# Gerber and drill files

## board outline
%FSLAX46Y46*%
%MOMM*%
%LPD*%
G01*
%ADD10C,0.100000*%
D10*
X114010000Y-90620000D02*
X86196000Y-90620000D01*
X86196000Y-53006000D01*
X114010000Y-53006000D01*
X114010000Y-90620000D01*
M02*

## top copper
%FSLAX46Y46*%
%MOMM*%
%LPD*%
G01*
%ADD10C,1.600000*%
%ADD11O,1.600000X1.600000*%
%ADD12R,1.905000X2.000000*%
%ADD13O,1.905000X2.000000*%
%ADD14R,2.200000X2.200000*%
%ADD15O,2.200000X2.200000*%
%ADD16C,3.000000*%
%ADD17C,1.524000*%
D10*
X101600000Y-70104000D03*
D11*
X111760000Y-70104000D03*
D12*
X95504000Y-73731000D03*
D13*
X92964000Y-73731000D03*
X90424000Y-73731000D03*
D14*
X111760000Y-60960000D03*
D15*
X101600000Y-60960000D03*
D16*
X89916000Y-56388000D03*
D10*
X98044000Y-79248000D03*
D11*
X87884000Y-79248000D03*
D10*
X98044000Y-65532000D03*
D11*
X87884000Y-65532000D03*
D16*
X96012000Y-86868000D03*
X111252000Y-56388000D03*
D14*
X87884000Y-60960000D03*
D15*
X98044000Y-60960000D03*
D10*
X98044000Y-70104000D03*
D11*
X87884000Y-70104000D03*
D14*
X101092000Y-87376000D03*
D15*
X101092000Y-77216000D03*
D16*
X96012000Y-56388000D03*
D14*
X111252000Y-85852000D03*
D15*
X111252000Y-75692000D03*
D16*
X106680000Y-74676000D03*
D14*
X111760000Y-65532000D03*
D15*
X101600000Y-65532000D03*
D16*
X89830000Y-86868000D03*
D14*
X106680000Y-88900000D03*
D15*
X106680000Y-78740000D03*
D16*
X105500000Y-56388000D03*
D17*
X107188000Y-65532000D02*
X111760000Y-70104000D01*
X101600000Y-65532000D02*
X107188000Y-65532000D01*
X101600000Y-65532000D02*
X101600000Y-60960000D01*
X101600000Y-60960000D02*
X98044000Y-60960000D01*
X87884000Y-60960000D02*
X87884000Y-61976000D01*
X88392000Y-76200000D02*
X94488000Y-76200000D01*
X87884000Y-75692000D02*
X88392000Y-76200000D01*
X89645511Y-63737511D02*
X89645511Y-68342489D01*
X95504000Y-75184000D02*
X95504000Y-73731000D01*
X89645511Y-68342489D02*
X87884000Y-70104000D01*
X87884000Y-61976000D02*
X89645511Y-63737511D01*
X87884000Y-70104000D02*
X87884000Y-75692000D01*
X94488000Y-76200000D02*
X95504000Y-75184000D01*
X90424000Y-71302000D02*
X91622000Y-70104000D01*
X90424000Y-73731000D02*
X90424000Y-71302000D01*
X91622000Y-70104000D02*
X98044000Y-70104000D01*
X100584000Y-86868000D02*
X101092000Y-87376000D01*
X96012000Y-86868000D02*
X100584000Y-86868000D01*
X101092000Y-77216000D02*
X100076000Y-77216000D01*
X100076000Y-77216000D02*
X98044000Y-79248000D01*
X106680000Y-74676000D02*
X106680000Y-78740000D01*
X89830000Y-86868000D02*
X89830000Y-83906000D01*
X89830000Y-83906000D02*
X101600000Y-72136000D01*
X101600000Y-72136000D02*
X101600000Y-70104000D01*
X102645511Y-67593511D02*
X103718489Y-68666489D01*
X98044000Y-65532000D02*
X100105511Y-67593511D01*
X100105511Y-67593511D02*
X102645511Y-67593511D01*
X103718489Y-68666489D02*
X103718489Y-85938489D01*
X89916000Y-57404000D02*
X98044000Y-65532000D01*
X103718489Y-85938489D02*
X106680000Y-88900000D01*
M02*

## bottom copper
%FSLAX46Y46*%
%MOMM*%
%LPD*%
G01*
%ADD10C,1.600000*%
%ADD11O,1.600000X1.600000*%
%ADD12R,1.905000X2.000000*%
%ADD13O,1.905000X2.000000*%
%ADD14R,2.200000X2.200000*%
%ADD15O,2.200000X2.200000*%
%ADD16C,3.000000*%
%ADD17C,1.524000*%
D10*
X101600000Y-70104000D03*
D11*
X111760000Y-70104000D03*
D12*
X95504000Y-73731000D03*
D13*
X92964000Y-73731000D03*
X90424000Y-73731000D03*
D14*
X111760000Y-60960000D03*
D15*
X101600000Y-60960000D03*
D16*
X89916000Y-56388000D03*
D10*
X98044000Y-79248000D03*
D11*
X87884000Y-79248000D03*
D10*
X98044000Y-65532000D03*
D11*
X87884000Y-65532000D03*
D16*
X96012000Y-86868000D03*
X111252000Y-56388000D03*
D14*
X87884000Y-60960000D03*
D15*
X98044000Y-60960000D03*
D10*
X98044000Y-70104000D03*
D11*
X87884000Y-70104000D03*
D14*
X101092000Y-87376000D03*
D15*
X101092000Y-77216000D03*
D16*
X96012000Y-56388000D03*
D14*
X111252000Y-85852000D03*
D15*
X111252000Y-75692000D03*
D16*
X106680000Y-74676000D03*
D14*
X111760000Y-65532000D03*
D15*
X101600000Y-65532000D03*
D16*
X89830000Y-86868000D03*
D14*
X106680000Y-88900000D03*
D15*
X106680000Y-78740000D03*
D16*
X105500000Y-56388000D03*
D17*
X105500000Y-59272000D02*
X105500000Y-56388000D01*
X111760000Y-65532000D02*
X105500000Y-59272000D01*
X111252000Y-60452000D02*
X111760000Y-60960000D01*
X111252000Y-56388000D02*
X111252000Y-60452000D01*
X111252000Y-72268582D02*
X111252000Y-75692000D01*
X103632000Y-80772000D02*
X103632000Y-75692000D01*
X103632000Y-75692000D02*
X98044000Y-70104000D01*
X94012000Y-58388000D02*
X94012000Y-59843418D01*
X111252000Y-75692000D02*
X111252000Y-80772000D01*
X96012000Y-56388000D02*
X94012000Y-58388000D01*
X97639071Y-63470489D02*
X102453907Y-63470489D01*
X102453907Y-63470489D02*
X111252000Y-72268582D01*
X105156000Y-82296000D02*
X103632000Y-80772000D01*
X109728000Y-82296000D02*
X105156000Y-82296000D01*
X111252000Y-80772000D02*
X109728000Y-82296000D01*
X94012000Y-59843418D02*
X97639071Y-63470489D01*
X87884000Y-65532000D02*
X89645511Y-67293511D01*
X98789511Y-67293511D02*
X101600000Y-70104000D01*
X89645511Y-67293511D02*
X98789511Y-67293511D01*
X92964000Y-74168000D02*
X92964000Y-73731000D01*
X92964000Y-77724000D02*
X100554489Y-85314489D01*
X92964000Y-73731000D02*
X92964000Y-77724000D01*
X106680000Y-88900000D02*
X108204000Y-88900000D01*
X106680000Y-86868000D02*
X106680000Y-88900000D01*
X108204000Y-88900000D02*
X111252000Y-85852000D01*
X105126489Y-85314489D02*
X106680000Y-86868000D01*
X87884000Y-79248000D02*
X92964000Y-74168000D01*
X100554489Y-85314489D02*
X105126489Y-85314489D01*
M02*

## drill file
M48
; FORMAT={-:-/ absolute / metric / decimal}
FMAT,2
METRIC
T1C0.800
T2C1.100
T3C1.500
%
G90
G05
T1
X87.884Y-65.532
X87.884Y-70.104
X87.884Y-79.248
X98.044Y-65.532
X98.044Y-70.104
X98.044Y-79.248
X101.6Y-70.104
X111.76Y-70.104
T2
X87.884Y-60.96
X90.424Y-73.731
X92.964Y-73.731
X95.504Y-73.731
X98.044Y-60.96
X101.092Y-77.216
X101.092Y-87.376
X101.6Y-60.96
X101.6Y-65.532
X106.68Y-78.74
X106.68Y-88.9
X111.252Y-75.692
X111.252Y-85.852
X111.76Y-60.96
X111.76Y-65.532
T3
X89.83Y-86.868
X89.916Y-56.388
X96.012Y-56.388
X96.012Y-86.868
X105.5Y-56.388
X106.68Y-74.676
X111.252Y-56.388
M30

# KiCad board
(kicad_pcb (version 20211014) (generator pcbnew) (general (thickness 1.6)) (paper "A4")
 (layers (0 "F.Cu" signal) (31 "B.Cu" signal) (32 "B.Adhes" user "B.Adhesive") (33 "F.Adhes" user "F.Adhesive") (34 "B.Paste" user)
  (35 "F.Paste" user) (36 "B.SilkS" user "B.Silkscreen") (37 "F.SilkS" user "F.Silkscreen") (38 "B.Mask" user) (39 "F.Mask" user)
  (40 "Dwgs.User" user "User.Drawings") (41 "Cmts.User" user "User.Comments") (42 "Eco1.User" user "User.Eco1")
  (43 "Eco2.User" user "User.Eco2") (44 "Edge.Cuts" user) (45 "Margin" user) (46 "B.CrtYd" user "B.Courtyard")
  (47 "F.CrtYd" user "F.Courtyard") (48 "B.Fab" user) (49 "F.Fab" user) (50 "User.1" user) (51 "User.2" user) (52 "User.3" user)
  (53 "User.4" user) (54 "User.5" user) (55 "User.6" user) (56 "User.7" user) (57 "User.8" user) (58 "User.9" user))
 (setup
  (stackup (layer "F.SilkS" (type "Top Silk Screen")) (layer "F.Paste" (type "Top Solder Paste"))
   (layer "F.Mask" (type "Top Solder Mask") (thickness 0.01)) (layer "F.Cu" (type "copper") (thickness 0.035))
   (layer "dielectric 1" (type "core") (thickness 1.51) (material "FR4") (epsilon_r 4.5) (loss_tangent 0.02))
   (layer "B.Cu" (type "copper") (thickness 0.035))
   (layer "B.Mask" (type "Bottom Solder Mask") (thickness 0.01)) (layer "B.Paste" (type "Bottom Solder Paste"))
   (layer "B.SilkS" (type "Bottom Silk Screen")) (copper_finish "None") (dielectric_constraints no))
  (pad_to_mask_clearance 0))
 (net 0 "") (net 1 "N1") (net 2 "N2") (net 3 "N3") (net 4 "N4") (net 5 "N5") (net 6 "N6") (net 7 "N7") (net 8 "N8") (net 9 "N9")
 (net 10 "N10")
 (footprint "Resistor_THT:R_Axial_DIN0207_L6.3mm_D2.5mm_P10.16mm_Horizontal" (layer "F.Cu") (at 101.6 70.104)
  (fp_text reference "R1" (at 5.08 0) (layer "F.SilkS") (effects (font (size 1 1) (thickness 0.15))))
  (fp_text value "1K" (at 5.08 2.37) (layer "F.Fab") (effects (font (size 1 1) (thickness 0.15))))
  (pad "1" thru_hole circle (at 0 0) (size 1.6 1.6) (drill 0.8) (layers *.Cu *.Mask) (remove_unused_layers) (keep_end_layers) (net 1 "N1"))
  (pad "2" thru_hole oval (at 10.16 0) (size 1.6 1.6) (drill 0.8) (layers *.Cu *.Mask) (remove_unused_layers) (keep_end_layers) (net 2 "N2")))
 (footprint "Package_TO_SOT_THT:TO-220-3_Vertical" (layer "F.Cu") (at 95.504 73.731 180)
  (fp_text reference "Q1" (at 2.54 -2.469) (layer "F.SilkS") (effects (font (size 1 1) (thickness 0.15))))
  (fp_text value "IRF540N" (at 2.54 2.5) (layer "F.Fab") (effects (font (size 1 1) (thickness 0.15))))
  (pad "1" thru_hole rect (at 0 0 180) (size 1.905 2) (drill 1.1) (layers *.Cu *.Mask) (remove_unused_layers) (keep_end_layers) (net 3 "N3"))
  (pad "2" thru_hole oval (at 2.54 0 180) (size 1.905 2) (drill 1.1) (layers *.Cu *.Mask) (remove_unused_layers) (keep_end_layers)
   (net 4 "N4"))
  (pad "3" thru_hole oval (at 5.08 0 180) (size 1.905 2) (drill 1.1) (layers *.Cu *.Mask) (remove_unused_layers) (keep_end_layers)
   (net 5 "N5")))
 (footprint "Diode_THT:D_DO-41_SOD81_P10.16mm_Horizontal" (layer "F.Cu") (at 111.76 60.96 180)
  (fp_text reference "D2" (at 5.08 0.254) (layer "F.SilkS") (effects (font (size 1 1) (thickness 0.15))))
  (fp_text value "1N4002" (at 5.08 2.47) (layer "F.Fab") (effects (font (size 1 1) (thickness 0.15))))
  (pad "1" thru_hole rect (at 0 0 180) (size 2.2 2.2) (drill 1.1) (layers *.Cu *.Mask) (remove_unused_layers) (keep_end_layers) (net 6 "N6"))
  (pad "2" thru_hole oval (at 10.16 0 180) (size 2.2 2.2) (drill 1.1) (layers *.Cu *.Mask) (remove_unused_layers) (keep_end_layers)
   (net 2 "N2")))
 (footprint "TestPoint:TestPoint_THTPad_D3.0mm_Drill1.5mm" (layer "F.Cu") (at 89.916 56.388)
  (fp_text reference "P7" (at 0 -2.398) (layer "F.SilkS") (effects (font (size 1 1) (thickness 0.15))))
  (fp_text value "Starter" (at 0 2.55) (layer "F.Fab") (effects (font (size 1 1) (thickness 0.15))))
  (pad "1" thru_hole circle (at 0 0) (size 3 3) (drill 1.5) (layers *.Cu *.Mask) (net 4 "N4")))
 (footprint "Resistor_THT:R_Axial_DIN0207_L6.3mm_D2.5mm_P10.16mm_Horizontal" (layer "F.Cu") (at 98.044 79.248 180)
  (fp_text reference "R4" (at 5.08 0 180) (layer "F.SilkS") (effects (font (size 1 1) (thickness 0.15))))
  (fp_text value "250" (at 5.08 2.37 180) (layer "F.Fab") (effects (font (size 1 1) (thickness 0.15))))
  (pad "1" thru_hole circle (at 0 0 180) (size 1.6 1.6) (drill 0.8) (layers *.Cu *.Mask) (remove_unused_layers) (keep_end_layers)
   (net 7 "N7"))
  (pad "2" thru_hole oval (at 10.16 0 180) (size 1.6 1.6) (drill 0.8) (layers *.Cu *.Mask) (remove_unused_layers) (keep_end_layers)
   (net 4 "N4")))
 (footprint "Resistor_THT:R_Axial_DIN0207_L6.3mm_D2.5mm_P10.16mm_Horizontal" (layer "F.Cu") (at 98.044 65.532 180)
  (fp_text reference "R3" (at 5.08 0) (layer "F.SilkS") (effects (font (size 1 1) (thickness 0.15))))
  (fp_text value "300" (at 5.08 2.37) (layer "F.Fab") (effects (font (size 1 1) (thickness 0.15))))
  (pad "1" thru_hole circle (at 0 0 180) (size 1.6 1.6) (drill 0.8) (layers *.Cu *.Mask) (remove_unused_layers) (keep_end_layers)
   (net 4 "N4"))
  (pad "2" thru_hole oval (at 10.16 0 180) (size 1.6 1.6) (drill 0.8) (layers *.Cu *.Mask) (remove_unused_layers) (keep_end_layers)
   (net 1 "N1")))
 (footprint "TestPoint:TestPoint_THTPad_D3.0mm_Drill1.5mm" (layer "F.Cu") (at 96.012 86.868)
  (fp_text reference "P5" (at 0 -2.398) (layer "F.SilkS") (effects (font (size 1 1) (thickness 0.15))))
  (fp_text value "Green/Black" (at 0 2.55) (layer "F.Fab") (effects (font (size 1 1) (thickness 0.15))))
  (pad "1" thru_hole circle (at 0 0) (size 3 3) (drill 1.5) (layers *.Cu *.Mask) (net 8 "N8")))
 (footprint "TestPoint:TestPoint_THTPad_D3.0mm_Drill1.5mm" (layer "F.Cu") (at 111.252 56.388)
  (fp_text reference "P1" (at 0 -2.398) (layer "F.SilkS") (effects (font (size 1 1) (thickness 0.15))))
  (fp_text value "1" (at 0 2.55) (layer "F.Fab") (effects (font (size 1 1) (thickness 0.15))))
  (pad "1" thru_hole circle (at 0 0) (size 3 3) (drill 1.5) (layers *.Cu *.Mask) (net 6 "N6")))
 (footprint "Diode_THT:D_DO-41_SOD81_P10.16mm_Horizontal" (layer "F.Cu") (at 87.884 60.96)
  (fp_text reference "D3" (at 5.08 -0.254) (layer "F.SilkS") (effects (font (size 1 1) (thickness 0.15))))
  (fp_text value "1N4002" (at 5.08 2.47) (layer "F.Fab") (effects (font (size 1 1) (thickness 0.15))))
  (pad "1" thru_hole rect (at 0 0) (size 2.2 2.2) (drill 1.1) (layers *.Cu *.Mask) (remove_unused_layers) (keep_end_layers) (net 3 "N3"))
  (pad "2" thru_hole oval (at 10.16 0) (size 2.2 2.2) (drill 1.1) (layers *.Cu *.Mask) (remove_unused_layers) (keep_end_layers) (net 2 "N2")))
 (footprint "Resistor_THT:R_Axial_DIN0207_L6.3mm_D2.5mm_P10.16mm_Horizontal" (layer "F.Cu") (at 98.044 70.104 180)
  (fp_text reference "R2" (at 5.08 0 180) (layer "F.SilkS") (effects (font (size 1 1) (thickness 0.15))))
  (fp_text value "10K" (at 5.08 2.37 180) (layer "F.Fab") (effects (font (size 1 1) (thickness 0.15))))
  (pad "1" thru_hole circle (at 0 0 180) (size 1.6 1.6) (drill 0.8) (layers *.Cu *.Mask) (remove_unused_layers) (keep_end_layers)
   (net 5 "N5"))
  (pad "2" thru_hole oval (at 10.16 0 180) (size 1.6 1.6) (drill 0.8) (layers *.Cu *.Mask) (remove_unused_layers) (keep_end_layers)
   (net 3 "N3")))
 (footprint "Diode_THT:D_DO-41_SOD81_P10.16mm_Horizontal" (layer "F.Cu") (at 101.092 87.376 90)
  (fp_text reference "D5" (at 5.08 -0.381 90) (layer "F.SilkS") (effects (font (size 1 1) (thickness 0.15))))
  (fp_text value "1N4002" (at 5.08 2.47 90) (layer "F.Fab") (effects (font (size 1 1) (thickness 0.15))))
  (pad "1" thru_hole rect (at 0 0 90) (size 2.2 2.2) (drill 1.1) (layers *.Cu *.Mask) (remove_unused_layers) (keep_end_layers) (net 8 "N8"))
  (pad "2" thru_hole oval (at 10.16 0 90) (size 2.2 2.2) (drill 1.1) (layers *.Cu *.Mask) (remove_unused_layers) (keep_end_layers)
   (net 7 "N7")))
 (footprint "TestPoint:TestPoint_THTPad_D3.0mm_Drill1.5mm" (layer "F.Cu") (at 96.012 56.388)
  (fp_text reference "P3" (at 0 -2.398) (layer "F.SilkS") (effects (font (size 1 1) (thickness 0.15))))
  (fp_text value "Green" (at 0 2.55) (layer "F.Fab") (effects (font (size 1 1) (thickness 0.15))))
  (pad "1" thru_hole circle (at 0 0) (size 3 3) (drill 1.5) (layers *.Cu *.Mask) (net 5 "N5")))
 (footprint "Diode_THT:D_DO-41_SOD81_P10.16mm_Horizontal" (layer "F.Cu") (at 111.252 85.852 90)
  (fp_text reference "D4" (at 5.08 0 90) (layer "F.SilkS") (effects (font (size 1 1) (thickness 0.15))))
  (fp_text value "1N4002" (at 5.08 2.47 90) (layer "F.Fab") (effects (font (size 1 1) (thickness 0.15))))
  (pad "1" thru_hole rect (at 0 0 90) (size 2.2 2.2) (drill 1.1) (layers *.Cu *.Mask) (remove_unused_layers) (keep_end_layers) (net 4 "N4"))
  (pad "2" thru_hole oval (at 10.16 0 90) (size 2.2 2.2) (drill 1.1) (layers *.Cu *.Mask) (remove_unused_layers) (keep_end_layers)
   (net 5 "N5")))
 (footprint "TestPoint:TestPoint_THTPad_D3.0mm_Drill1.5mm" (layer "F.Cu") (at 106.68 74.676)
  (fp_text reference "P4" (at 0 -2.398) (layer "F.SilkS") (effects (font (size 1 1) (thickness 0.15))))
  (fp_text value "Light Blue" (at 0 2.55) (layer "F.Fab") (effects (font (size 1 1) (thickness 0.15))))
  (pad "1" thru_hole circle (at 0 0) (size 3 3) (drill 1.5) (layers *.Cu *.Mask) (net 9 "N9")))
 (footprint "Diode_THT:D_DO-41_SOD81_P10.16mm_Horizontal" (layer "F.Cu") (at 111.76 65.532 180)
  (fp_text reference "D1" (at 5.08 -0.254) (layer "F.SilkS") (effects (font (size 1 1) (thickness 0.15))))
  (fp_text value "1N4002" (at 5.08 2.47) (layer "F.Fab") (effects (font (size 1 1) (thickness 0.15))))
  (pad "1" thru_hole rect (at 0 0 180) (size 2.2 2.2) (drill 1.1) (layers *.Cu *.Mask) (remove_unused_layers) (keep_end_layers)
   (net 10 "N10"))
  (pad "2" thru_hole oval (at 10.16 0 180) (size 2.2 2.2) (drill 1.1) (layers *.Cu *.Mask) (remove_unused_layers) (keep_end_layers)
   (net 2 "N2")))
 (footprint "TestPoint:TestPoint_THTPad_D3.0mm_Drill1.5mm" (layer "F.Cu") (at 89.83 86.868)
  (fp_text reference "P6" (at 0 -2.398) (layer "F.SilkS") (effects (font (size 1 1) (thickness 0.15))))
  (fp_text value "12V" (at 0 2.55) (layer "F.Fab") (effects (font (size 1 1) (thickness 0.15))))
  (pad "1" thru_hole circle (at 0 0) (size 3 3) (drill 1.5) (layers *.Cu *.Mask) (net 1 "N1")))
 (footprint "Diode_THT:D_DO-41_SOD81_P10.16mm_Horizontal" (layer "F.Cu") (at 106.68 88.9 90)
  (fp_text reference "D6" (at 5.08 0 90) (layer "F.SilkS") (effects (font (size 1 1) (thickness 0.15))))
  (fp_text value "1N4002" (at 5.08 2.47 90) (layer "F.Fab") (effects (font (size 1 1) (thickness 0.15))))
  (pad "1" thru_hole rect (at 0 0 90) (size 2.2 2.2) (drill 1.1) (layers *.Cu *.Mask) (remove_unused_layers) (keep_end_layers) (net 4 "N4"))
  (pad "2" thru_hole oval (at 10.16 0 90) (size 2.2 2.2) (drill 1.1) (layers *.Cu *.Mask) (remove_unused_layers) (keep_end_layers)
   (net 9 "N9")))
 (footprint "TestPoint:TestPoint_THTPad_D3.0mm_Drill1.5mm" (layer "F.Cu") (at 105.5 56.388)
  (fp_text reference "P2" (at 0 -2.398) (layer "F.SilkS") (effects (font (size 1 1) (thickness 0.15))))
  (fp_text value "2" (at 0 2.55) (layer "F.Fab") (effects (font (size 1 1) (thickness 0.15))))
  (pad "1" thru_hole circle (at 0 0) (size 3 3) (drill 1.5) (layers *.Cu *.Mask) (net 10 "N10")))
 (gr_poly (pts (xy 114.01 90.62) (xy 86.196 90.62) (xy 86.196 53.006) (xy 114.01 53.006)) (layer "Edge.Cuts") (width 0.1) (fill none))
 (segment (start 105.5 59.272) (end 105.5 56.388) (width 1.524) (layer "B.Cu") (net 10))
 (segment (start 111.76 65.532) (end 105.5 59.272) (width 1.524) (layer "B.Cu") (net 10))
 (segment (start 107.188 65.532) (end 111.76 70.104) (width 1.524) (layer "F.Cu") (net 2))
 (segment (start 101.6 65.532) (end 107.188 65.532) (width 1.524) (layer "F.Cu") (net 2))
 (segment (start 101.6 65.532) (end 101.6 60.96) (width 1.524) (layer "F.Cu") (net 2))
 (segment (start 101.6 60.96) (end 98.044 60.96) (width 1.524) (layer "F.Cu") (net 2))
 (segment (start 111.252 60.452) (end 111.76 60.96) (width 1.524) (layer "B.Cu") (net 6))
 (segment (start 111.252 56.388) (end 111.252 60.452) (width 1.524) (layer "B.Cu") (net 6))
 (segment (start 87.884 60.96) (end 87.884 61.976) (width 1.524) (layer "F.Cu") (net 3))
 (segment (start 88.392 76.2) (end 94.488 76.2) (width 1.524) (layer "F.Cu") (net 3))
 (segment (start 87.884 75.692) (end 88.392 76.2) (width 1.524) (layer "F.Cu") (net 3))
 (segment (start 89.645511 63.737511) (end 89.645511 68.342489) (width 1.524) (layer "F.Cu") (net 3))
 (segment (start 95.504 75.184) (end 95.504 73.731) (width 1.524) (layer "F.Cu") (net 3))
 (segment (start 89.645511 68.342489) (end 87.884 70.104) (width 1.524) (layer "F.Cu") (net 3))
 (segment (start 87.884 61.976) (end 89.645511 63.737511) (width 1.524) (layer "F.Cu") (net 3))
 (segment (start 87.884 70.104) (end 87.884 75.692) (width 1.524) (layer "F.Cu") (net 3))
 (segment (start 94.488 76.2) (end 95.504 75.184) (width 1.524) (layer "F.Cu") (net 3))
 (segment (start 90.424 71.302) (end 91.622 70.104) (width 1.524) (layer "F.Cu") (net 5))
 (segment (start 90.424 73.731) (end 90.424 71.302) (width 1.524) (layer "F.Cu") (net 5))
 (segment (start 91.622 70.104) (end 98.044 70.104) (width 1.524) (layer "F.Cu") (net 5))
 (segment (start 111.252 72.268582) (end 111.252 75.692) (width 1.524) (layer "B.Cu") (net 5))
 (segment (start 103.632 80.772) (end 103.632 75.692) (width 1.524) (layer "B.Cu") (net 5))
 (segment (start 103.632 75.692) (end 98.044 70.104) (width 1.524) (layer "B.Cu") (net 5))
 (segment (start 94.012 58.388) (end 94.012 59.843418) (width 1.524) (layer "B.Cu") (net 5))
 (segment (start 111.252 75.692) (end 111.252 80.772) (width 1.524) (layer "B.Cu") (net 5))
 (segment (start 96.012 56.388) (end 94.012 58.388) (width 1.524) (layer "B.Cu") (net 5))
 (segment (start 97.639071 63.470489) (end 102.453907 63.470489) (width 1.524) (layer "B.Cu") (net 5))
 (segment (start 102.453907 63.470489) (end 111.252 72.268582) (width 1.524) (layer "B.Cu") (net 5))
 (segment (start 105.156 82.296) (end 103.632 80.772) (width 1.524) (layer "B.Cu") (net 5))
 (segment (start 109.728 82.296) (end 105.156 82.296) (width 1.524) (layer "B.Cu") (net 5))
 (segment (start 111.252 80.772) (end 109.728 82.296) (width 1.524) (layer "B.Cu") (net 5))
 (segment (start 94.012 59.843418) (end 97.639071 63.470489) (width 1.524) (layer "B.Cu") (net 5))
 (segment (start 100.584 86.868) (end 101.092 87.376) (width 1.524) (layer "F.Cu") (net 8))
 (segment (start 96.012 86.868) (end 100.584 86.868) (width 1.524) (layer "F.Cu") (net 8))
 (segment (start 101.092 77.216) (end 100.076 77.216) (width 1.524) (layer "F.Cu") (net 7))
 (segment (start 100.076 77.216) (end 98.044 79.248) (width 1.524) (layer "F.Cu") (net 7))
 (segment (start 106.68 74.676) (end 106.68 78.74) (width 1.524) (layer "F.Cu") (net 9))
 (segment (start 89.83 86.868) (end 89.83 83.906) (width 1.524) (layer "F.Cu") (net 1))
 (segment (start 89.83 83.906) (end 101.6 72.136) (width 1.524) (layer "F.Cu") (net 1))
 (segment (start 101.6 72.136) (end 101.6 70.104) (width 1.524) (layer "F.Cu") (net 1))
 (segment (start 87.884 65.532) (end 89.645511 67.293511) (width 1.524) (layer "B.Cu") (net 1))
 (segment (start 98.789511 67.293511) (end 101.6 70.104) (width 1.524) (layer "B.Cu") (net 1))
 (segment (start 89.645511 67.293511) (end 98.789511 67.293511) (width 1.524) (layer "B.Cu") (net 1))
 (segment (start 102.645511 67.593511) (end 103.718489 68.666489) (width 1.524) (layer "F.Cu") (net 4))
 (segment (start 98.044 65.532) (end 100.105511 67.593511) (width 1.524) (layer "F.Cu") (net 4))
 (segment (start 100.105511 67.593511) (end 102.645511 67.593511) (width 1.524) (layer "F.Cu") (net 4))
 (segment (start 103.718489 68.666489) (end 103.718489 85.938489) (width 1.524) (layer "F.Cu") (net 4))
 (segment (start 89.916 57.404) (end 98.044 65.532) (width 1.524) (layer "F.Cu") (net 4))
 (segment (start 103.718489 85.938489) (end 106.68 88.9) (width 1.524) (layer "F.Cu") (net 4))
 (segment (start 92.964 74.168) (end 92.964 73.731) (width 1.524) (layer "B.Cu") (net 4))
 (segment (start 92.964 77.724) (end 100.554489 85.314489) (width 1.524) (layer "B.Cu") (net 4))
 (segment (start 92.964 73.731) (end 92.964 77.724) (width 1.524) (layer "B.Cu") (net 4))
 (segment (start 106.68 88.9) (end 108.204 88.9) (width 1.524) (layer "B.Cu") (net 4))
 (segment (start 106.68 86.868) (end 106.68 88.9) (width 1.524) (layer "B.Cu") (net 4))
 (segment (start 108.204 88.9) (end 111.252 85.852) (width 1.524) (layer "B.Cu") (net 4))
 (segment (start 105.126489 85.314489) (end 106.68 86.868) (width 1.524) (layer "B.Cu") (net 4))
 (segment (start 87.884 79.248) (end 92.964 74.168) (width 1.524) (layer "B.Cu") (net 4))
 (segment (start 100.554489 85.314489) (end 105.126489 85.314489) (width 1.524) (layer "B.Cu") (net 4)))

